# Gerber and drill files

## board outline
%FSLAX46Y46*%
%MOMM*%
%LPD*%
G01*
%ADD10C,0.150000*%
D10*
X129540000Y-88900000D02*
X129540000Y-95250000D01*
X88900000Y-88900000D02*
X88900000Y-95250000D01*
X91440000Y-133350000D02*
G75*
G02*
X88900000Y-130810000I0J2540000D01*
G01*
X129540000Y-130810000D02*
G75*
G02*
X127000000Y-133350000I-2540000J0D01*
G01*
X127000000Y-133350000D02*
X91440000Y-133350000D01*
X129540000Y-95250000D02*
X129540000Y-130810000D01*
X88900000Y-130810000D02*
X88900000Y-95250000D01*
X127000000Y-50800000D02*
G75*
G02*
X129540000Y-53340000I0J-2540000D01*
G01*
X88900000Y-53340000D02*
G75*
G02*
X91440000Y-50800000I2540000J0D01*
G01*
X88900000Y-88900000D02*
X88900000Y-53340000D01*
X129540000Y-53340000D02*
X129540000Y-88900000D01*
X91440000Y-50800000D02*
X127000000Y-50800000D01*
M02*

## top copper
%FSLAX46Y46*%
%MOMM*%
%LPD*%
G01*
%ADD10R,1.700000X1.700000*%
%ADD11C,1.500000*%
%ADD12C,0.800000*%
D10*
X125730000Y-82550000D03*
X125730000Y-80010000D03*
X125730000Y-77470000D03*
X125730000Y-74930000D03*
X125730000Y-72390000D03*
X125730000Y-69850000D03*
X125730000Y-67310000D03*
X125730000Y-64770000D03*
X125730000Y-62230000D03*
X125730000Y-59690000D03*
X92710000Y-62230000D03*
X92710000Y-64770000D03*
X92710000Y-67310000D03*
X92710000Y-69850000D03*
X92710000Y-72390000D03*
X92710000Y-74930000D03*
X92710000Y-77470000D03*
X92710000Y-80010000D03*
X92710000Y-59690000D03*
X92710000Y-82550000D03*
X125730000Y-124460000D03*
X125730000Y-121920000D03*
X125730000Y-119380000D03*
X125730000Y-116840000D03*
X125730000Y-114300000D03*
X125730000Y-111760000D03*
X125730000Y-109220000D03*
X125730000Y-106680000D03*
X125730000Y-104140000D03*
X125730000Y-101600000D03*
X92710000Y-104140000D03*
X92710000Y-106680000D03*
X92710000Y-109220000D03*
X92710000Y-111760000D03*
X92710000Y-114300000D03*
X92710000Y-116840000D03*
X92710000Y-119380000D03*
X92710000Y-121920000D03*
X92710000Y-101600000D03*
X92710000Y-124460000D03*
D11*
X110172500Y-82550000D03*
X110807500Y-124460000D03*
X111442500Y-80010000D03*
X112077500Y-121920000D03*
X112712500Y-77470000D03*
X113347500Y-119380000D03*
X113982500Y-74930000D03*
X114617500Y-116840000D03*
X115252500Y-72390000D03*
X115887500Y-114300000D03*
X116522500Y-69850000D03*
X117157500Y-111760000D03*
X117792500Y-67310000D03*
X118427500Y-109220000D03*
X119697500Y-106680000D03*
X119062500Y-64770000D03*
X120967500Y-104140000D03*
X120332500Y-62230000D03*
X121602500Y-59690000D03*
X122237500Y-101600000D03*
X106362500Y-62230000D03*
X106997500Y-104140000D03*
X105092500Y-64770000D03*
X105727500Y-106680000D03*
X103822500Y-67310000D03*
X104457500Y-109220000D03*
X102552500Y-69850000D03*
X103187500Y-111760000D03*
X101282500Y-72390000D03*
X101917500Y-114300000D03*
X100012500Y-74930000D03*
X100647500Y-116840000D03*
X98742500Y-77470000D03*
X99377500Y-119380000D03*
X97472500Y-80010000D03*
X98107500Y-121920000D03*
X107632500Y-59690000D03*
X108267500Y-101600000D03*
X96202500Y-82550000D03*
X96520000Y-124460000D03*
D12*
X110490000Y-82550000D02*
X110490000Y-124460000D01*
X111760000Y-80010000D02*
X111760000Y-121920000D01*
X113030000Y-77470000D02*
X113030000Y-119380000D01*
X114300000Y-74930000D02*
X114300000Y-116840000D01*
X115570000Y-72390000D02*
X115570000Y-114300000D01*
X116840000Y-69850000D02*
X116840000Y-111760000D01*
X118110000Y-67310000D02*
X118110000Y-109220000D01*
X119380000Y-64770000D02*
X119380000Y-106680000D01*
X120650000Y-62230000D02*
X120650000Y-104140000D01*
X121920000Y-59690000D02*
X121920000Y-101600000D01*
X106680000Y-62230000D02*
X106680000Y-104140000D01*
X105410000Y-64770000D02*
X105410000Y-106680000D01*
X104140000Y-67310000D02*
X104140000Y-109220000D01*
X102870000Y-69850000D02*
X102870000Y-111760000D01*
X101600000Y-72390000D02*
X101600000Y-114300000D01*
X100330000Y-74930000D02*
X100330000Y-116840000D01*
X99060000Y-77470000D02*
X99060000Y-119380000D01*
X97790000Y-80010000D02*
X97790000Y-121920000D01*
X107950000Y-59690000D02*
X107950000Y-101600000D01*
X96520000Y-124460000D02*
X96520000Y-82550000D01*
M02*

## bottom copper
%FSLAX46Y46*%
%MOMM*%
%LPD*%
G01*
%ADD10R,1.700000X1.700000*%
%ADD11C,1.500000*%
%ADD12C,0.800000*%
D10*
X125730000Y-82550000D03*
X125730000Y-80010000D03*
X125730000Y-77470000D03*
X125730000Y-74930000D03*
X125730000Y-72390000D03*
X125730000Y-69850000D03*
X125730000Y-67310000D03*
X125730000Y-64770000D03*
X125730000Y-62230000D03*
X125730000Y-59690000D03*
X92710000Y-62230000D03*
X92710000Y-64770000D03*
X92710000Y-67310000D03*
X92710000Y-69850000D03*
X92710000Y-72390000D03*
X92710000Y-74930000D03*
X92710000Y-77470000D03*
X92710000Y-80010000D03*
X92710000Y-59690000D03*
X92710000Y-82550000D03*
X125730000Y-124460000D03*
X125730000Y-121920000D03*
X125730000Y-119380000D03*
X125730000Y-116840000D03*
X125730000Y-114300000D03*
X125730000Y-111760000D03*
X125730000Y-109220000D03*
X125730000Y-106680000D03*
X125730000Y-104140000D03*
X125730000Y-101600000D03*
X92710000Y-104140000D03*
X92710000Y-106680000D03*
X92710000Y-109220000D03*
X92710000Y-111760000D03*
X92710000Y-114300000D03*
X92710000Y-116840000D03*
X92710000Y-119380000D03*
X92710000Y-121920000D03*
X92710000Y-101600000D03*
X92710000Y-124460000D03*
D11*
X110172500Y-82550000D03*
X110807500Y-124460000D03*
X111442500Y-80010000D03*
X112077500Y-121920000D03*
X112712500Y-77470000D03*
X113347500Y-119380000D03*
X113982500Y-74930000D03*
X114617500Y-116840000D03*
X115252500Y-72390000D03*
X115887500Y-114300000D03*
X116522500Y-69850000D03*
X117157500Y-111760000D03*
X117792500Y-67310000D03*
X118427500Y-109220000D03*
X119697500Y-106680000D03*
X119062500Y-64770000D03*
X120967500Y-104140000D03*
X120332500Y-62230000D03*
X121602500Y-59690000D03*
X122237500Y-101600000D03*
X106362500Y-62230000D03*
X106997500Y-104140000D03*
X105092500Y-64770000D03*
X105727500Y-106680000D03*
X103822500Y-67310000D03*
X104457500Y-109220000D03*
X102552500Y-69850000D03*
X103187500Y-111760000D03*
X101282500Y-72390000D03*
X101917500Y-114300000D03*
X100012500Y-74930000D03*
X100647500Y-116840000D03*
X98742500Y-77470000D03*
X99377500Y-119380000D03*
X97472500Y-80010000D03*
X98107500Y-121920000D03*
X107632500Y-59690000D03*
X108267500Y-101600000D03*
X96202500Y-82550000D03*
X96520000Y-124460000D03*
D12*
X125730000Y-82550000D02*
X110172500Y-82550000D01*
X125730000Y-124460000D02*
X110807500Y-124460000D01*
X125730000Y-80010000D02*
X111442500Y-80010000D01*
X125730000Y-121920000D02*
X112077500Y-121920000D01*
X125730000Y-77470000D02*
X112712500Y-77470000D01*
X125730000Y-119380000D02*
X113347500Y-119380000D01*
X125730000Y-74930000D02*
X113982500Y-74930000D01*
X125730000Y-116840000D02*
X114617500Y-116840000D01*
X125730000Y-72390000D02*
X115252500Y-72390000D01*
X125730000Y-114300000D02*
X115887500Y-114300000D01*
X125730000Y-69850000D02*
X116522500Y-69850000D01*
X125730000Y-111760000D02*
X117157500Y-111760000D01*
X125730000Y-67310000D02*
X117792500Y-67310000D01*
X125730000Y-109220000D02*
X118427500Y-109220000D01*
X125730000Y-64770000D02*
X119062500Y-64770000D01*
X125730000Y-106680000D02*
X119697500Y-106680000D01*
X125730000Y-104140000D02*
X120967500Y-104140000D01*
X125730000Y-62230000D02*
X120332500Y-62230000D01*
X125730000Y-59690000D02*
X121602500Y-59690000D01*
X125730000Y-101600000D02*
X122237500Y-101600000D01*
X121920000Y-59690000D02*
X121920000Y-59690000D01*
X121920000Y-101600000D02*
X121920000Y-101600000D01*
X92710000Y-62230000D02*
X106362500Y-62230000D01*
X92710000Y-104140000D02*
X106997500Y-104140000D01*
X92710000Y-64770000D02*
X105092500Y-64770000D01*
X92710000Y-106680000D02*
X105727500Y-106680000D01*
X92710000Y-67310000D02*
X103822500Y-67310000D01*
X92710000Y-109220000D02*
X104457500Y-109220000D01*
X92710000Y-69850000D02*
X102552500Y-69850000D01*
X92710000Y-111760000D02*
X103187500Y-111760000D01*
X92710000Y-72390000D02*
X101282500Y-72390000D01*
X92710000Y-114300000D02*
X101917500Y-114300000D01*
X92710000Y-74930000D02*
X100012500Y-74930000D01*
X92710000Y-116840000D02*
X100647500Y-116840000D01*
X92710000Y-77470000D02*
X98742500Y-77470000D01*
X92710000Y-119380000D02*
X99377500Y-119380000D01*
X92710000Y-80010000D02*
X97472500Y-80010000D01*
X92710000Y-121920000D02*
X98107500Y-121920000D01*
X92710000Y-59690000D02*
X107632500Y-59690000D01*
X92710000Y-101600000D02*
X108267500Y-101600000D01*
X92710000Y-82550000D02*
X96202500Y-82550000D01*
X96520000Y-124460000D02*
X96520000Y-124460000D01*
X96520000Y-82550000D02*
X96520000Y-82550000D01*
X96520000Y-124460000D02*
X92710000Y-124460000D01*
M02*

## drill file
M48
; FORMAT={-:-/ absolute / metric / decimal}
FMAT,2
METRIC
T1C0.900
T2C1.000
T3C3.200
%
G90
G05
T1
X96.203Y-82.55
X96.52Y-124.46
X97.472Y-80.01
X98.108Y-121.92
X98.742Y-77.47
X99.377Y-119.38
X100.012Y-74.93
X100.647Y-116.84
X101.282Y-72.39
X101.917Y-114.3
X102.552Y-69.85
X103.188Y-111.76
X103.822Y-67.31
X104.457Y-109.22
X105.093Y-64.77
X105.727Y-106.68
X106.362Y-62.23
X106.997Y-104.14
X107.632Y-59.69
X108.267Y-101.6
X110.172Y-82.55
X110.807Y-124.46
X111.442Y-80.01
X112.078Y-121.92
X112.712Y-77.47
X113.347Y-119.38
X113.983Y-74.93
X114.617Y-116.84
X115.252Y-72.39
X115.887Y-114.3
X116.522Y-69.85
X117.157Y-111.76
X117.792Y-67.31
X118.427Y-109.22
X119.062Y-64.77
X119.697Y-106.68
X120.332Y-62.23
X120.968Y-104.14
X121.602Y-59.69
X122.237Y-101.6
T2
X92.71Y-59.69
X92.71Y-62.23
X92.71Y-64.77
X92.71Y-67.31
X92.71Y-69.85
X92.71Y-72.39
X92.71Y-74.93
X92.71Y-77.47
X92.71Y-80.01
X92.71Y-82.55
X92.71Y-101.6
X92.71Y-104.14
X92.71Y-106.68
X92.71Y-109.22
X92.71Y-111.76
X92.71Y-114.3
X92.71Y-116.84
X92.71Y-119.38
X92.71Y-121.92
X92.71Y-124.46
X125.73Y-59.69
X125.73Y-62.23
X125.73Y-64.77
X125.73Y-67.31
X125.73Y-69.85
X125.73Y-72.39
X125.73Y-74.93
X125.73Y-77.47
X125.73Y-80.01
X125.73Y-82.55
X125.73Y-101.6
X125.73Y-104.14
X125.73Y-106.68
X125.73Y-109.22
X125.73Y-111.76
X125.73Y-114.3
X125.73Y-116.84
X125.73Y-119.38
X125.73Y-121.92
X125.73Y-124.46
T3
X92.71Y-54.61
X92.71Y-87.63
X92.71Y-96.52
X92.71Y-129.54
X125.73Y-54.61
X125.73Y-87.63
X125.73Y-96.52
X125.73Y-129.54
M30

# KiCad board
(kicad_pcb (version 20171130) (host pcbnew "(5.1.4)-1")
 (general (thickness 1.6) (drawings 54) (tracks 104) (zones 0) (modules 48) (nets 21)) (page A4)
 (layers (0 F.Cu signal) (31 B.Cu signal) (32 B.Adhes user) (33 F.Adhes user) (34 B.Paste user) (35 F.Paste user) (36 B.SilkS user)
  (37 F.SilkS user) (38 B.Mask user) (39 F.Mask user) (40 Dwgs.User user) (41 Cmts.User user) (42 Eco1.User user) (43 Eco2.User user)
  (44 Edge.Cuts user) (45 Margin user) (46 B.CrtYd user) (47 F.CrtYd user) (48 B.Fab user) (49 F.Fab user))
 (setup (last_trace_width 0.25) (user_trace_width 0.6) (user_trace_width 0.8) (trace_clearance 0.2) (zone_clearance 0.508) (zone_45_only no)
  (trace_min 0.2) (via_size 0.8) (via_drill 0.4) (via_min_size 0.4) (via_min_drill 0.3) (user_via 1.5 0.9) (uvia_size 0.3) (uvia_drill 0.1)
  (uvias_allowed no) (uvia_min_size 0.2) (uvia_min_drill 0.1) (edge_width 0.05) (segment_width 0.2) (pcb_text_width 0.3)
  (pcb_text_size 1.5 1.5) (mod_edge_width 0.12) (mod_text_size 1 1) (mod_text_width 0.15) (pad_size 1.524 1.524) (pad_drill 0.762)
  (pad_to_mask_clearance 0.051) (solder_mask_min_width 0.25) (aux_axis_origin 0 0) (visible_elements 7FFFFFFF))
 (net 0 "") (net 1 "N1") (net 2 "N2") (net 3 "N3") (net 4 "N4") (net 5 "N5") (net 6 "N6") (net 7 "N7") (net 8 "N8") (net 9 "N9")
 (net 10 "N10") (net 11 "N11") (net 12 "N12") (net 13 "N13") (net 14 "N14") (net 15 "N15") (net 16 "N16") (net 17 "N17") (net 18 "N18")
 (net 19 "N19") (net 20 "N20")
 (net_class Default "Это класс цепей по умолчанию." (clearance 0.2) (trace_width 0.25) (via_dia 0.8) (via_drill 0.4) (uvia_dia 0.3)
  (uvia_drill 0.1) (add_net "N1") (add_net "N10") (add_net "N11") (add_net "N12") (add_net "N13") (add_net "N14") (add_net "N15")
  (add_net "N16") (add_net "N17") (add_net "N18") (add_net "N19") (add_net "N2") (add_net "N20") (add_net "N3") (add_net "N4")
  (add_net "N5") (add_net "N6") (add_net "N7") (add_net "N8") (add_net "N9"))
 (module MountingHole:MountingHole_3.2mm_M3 (layer F.Cu) (at 92.71 129.54)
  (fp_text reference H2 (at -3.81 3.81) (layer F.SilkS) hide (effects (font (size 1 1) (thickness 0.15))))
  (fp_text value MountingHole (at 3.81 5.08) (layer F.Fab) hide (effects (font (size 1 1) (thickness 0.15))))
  (pad 1 np_thru_hole circle (at 0 0) (size 3.2 3.2) (drill 3.2) (layers *.Cu *.Mask)))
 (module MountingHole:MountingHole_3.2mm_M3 (layer F.Cu) (at 125.73 129.54)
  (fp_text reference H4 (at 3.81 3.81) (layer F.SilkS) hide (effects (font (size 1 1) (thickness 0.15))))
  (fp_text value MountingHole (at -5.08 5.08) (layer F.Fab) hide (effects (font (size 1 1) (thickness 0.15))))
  (pad 1 np_thru_hole circle (at 0 0) (size 3.2 3.2) (drill 3.2) (layers *.Cu *.Mask)))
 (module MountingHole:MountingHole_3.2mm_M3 (layer F.Cu) (at 92.71 96.52)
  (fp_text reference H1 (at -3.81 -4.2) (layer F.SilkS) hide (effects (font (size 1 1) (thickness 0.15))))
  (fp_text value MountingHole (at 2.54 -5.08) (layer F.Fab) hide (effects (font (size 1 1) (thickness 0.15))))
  (pad 1 np_thru_hole circle (at 0 0) (size 3.2 3.2) (drill 3.2) (layers *.Cu *.Mask)))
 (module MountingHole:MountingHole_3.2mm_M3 (layer F.Cu) (at 125.73 96.52)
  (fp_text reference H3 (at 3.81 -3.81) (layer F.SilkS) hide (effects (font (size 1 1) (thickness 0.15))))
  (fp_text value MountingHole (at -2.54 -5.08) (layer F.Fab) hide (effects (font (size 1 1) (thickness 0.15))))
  (pad 1 np_thru_hole circle (at 0 0) (size 3.2 3.2) (drill 3.2) (layers *.Cu *.Mask)))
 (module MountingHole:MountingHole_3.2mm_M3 (layer F.Cu) (at 92.71 54.61)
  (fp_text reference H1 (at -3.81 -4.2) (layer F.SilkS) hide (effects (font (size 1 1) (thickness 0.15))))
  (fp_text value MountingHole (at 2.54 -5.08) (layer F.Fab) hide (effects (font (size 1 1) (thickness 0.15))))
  (pad 1 np_thru_hole circle (at 0 0) (size 3.2 3.2) (drill 3.2) (layers *.Cu *.Mask)))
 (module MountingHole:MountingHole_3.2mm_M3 (layer F.Cu) (at 92.71 87.63)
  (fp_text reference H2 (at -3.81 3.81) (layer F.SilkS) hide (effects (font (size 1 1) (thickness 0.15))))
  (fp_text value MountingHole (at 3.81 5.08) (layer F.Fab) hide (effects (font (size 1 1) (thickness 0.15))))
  (pad 1 np_thru_hole circle (at 0 0) (size 3.2 3.2) (drill 3.2) (layers *.Cu *.Mask)))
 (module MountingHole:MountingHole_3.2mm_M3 (layer F.Cu) (at 125.73 54.61)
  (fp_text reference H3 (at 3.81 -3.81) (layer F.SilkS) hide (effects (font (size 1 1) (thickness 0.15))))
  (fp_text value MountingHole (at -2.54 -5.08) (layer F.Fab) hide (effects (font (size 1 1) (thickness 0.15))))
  (pad 1 np_thru_hole circle (at 0 0) (size 3.2 3.2) (drill 3.2) (layers *.Cu *.Mask)))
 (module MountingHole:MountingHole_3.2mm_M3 (layer F.Cu) (at 125.73 87.63)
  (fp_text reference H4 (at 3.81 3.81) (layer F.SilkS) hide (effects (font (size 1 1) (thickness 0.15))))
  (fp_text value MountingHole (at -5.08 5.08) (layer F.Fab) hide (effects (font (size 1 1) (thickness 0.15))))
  (pad 1 np_thru_hole circle (at 0 0) (size 3.2 3.2) (drill 3.2) (layers *.Cu *.Mask)))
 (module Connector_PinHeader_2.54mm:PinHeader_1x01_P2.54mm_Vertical (layer F.Cu) (at 125.73 82.55)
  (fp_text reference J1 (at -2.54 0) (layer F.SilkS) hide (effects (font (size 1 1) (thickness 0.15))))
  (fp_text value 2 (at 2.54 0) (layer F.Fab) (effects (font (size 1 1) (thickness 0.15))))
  (pad 1 thru_hole rect (at 0 0) (size 1.7 1.7) (drill 1) (layers *.Cu *.Mask) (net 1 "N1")))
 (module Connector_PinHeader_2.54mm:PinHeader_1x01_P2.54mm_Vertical (layer F.Cu) (at 125.73 80.01)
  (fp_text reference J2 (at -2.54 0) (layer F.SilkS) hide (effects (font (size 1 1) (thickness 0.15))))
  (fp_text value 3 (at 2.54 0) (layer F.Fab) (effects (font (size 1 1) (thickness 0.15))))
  (pad 1 thru_hole rect (at 0 0) (size 1.7 1.7) (drill 1) (layers *.Cu *.Mask) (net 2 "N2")))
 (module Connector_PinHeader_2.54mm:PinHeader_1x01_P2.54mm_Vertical (layer F.Cu) (at 125.73 77.47)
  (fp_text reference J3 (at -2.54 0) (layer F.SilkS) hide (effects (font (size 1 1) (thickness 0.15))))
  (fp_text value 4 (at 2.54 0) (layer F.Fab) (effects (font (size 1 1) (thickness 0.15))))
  (pad 1 thru_hole rect (at 0 0) (size 1.7 1.7) (drill 1) (layers *.Cu *.Mask) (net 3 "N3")))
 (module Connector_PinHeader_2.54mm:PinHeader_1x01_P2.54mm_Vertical (layer F.Cu) (at 125.73 74.93)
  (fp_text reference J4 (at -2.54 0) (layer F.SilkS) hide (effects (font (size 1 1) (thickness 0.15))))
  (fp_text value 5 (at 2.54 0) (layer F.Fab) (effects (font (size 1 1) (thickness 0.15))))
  (pad 1 thru_hole rect (at 0 0) (size 1.7 1.7) (drill 1) (layers *.Cu *.Mask) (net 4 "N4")))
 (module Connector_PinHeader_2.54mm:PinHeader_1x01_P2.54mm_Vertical (layer F.Cu) (at 125.73 72.39)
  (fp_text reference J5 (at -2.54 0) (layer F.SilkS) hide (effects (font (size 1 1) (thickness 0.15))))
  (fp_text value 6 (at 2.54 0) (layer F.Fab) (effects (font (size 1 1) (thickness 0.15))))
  (pad 1 thru_hole rect (at 0 0) (size 1.7 1.7) (drill 1) (layers *.Cu *.Mask) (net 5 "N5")))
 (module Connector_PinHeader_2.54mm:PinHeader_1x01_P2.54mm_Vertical (layer F.Cu) (at 125.73 69.85)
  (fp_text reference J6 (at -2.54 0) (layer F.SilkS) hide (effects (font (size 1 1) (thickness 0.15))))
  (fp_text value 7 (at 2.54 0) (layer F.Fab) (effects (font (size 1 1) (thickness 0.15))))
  (pad 1 thru_hole rect (at 0 0) (size 1.7 1.7) (drill 1) (layers *.Cu *.Mask) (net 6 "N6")))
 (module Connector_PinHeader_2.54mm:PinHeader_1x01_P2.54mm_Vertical (layer F.Cu) (at 125.73 67.31)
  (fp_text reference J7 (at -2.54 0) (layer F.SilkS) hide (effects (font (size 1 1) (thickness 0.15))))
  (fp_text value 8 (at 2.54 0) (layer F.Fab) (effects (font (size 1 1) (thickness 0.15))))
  (pad 1 thru_hole rect (at 0 0) (size 1.7 1.7) (drill 1) (layers *.Cu *.Mask) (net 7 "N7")))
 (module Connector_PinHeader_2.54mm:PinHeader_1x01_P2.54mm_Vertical (layer F.Cu) (at 125.73 64.77)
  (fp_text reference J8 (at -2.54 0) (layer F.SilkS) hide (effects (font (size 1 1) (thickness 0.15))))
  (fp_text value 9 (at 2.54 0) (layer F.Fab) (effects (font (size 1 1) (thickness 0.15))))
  (pad 1 thru_hole rect (at 0 0) (size 1.7 1.7) (drill 1) (layers *.Cu *.Mask) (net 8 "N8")))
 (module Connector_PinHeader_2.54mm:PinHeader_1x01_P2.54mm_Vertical (layer F.Cu) (at 125.73 62.23)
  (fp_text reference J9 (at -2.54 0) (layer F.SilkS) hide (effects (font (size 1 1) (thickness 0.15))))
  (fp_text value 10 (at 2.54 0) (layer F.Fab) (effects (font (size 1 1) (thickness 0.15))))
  (pad 1 thru_hole rect (at 0 0) (size 1.7 1.7) (drill 1) (layers *.Cu *.Mask) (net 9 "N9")))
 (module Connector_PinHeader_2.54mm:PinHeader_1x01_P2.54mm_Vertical (layer F.Cu) (at 125.73 59.69)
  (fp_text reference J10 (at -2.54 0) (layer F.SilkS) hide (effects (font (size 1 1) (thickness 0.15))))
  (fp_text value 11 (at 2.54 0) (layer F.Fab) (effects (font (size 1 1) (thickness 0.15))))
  (pad 1 thru_hole rect (at 0 0) (size 1.7 1.7) (drill 1) (layers *.Cu *.Mask) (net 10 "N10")))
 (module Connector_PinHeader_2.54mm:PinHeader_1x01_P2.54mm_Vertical (layer F.Cu) (at 92.71 62.23)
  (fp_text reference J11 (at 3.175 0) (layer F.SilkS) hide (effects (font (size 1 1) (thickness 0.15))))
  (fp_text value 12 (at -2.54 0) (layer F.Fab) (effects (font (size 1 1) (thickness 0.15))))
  (pad 1 thru_hole rect (at 0 0) (size 1.7 1.7) (drill 1) (layers *.Cu *.Mask) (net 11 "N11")))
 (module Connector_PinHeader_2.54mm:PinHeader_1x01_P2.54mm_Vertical (layer F.Cu) (at 92.71 64.77)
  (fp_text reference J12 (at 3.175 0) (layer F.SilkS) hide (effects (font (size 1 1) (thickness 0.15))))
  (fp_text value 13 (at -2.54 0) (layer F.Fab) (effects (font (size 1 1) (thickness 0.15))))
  (pad 1 thru_hole rect (at 0 0) (size 1.7 1.7) (drill 1) (layers *.Cu *.Mask) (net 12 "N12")))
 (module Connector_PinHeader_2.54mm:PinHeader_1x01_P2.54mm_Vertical (layer F.Cu) (at 92.71 67.31)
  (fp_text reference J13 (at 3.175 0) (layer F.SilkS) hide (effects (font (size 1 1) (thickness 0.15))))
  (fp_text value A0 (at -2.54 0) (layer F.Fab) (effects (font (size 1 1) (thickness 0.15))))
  (pad 1 thru_hole rect (at 0 0) (size 1.7 1.7) (drill 1) (layers *.Cu *.Mask) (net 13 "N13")))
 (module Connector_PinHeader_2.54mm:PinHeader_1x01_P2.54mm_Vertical (layer F.Cu) (at 92.71 69.85)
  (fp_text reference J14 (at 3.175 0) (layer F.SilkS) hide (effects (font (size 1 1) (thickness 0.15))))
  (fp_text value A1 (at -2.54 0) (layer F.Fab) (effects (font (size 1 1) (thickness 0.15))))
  (pad 1 thru_hole rect (at 0 0) (size 1.7 1.7) (drill 1) (layers *.Cu *.Mask) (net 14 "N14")))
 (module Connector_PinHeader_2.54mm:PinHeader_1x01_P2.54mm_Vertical (layer F.Cu) (at 92.71 72.39)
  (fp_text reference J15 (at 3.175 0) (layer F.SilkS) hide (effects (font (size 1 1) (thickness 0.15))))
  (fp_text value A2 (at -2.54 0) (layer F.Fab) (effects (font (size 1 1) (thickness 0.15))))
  (pad 1 thru_hole rect (at 0 0) (size 1.7 1.7) (drill 1) (layers *.Cu *.Mask) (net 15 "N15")))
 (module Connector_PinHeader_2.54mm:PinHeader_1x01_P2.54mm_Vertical (layer F.Cu) (at 92.71 74.93)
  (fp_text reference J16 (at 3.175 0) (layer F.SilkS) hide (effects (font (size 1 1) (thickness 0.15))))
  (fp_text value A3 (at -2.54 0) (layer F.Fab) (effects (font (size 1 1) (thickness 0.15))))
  (pad 1 thru_hole rect (at 0 0) (size 1.7 1.7) (drill 1) (layers *.Cu *.Mask) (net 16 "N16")))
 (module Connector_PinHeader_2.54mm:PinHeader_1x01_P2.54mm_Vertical (layer F.Cu) (at 92.71 77.47)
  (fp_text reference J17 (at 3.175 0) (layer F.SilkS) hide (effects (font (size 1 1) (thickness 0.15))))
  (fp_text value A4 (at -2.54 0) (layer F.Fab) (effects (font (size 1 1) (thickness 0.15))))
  (pad 1 thru_hole rect (at 0 0) (size 1.7 1.7) (drill 1) (layers *.Cu *.Mask) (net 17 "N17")))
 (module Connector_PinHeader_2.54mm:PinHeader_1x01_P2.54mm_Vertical (layer F.Cu) (at 92.71 80.01)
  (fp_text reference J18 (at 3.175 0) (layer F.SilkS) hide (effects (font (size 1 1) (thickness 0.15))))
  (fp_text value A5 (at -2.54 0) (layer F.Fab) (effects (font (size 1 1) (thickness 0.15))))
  (pad 1 thru_hole rect (at 0 0) (size 1.7 1.7) (drill 1) (layers *.Cu *.Mask) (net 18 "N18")))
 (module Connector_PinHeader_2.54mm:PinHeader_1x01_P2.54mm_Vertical (layer F.Cu) (at 92.71 59.69)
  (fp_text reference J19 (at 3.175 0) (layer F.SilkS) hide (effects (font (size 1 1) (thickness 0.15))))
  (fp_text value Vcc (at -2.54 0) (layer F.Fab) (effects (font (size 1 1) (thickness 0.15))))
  (pad 1 thru_hole rect (at 0 0) (size 1.7 1.7) (drill 1) (layers *.Cu *.Mask) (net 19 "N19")))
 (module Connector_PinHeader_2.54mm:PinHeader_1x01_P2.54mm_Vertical (layer F.Cu) (at 92.71 82.55)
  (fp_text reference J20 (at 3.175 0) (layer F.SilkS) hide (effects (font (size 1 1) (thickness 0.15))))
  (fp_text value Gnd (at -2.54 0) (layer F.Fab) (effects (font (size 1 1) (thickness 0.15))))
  (pad 1 thru_hole rect (at 0 0) (size 1.7 1.7) (drill 1) (layers *.Cu *.Mask) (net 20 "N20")))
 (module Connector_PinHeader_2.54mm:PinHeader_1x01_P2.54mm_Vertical (layer F.Cu) (at 125.73 124.46)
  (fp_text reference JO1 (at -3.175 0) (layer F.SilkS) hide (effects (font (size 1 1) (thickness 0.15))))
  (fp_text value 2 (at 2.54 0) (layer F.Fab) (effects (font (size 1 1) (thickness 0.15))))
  (pad 1 thru_hole rect (at 0 0) (size 1.7 1.7) (drill 1) (layers *.Cu *.Mask) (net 1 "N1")))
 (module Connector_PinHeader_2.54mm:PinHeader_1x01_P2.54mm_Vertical (layer F.Cu) (at 125.73 121.92)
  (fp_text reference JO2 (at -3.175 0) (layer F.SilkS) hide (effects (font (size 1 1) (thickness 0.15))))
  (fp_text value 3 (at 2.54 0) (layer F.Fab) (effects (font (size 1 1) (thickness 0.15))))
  (pad 1 thru_hole rect (at 0 0) (size 1.7 1.7) (drill 1) (layers *.Cu *.Mask) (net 2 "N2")))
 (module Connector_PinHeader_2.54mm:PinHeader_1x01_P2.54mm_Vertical (layer F.Cu) (at 125.73 119.38)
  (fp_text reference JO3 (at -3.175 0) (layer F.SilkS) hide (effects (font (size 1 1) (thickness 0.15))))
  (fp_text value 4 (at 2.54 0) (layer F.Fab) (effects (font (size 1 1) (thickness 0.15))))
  (pad 1 thru_hole rect (at 0 0) (size 1.7 1.7) (drill 1) (layers *.Cu *.Mask) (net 3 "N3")))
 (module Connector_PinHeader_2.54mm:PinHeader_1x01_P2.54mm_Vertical (layer F.Cu) (at 125.73 116.84)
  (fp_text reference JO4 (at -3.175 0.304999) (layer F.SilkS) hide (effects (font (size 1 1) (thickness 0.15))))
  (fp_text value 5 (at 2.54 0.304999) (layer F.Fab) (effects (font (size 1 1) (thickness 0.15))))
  (pad 1 thru_hole rect (at 0 0) (size 1.7 1.7) (drill 1) (layers *.Cu *.Mask) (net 4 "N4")))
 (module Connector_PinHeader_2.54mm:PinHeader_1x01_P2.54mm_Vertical (layer F.Cu) (at 125.73 114.3)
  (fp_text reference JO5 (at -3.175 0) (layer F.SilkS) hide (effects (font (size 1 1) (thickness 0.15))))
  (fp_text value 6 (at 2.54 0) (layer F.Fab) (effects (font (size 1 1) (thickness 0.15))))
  (pad 1 thru_hole rect (at 0 0) (size 1.7 1.7) (drill 1) (layers *.Cu *.Mask) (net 5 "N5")))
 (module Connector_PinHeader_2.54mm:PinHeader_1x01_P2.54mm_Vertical (layer F.Cu) (at 125.73 111.76)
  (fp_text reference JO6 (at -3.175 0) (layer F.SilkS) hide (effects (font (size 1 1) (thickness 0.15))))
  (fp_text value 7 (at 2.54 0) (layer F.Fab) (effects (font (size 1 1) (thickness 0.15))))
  (pad 1 thru_hole rect (at 0 0) (size 1.7 1.7) (drill 1) (layers *.Cu *.Mask) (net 6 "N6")))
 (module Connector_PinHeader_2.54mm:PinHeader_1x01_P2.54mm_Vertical (layer F.Cu) (at 125.73 109.22)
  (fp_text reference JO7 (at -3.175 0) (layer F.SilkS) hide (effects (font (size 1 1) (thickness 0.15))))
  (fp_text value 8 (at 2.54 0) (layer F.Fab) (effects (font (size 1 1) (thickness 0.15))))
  (pad 1 thru_hole rect (at 0 0) (size 1.7 1.7) (drill 1) (layers *.Cu *.Mask) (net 7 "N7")))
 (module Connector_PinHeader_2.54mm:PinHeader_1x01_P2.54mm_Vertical (layer F.Cu) (at 125.73 106.68)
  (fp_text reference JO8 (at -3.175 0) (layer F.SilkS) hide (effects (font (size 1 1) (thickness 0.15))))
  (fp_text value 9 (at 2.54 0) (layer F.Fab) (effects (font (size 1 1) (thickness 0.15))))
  (pad 1 thru_hole rect (at 0 0) (size 1.7 1.7) (drill 1) (layers *.Cu *.Mask) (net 8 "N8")))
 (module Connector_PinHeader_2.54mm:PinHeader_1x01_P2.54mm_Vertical (layer F.Cu) (at 125.73 104.14)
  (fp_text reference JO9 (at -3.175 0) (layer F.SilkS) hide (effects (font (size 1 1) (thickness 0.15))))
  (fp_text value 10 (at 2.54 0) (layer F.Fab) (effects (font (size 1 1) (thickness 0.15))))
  (pad 1 thru_hole rect (at 0 0) (size 1.7 1.7) (drill 1) (layers *.Cu *.Mask) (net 9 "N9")))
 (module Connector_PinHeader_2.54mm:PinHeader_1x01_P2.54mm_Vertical (layer F.Cu) (at 125.73 101.6)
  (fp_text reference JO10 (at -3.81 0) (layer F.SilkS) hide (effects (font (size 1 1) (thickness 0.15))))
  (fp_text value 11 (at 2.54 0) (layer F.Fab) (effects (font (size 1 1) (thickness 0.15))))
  (pad 1 thru_hole rect (at 0 0) (size 1.7 1.7) (drill 1) (layers *.Cu *.Mask) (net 10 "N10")))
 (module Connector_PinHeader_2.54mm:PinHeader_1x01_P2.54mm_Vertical (layer F.Cu) (at 92.71 104.14)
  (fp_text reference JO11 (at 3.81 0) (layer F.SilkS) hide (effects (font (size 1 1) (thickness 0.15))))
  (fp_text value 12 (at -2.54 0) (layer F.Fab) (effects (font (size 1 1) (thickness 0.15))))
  (pad 1 thru_hole rect (at 0 0) (size 1.7 1.7) (drill 1) (layers *.Cu *.Mask) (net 11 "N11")))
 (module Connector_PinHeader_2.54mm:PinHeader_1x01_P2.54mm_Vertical (layer F.Cu) (at 92.71 106.68)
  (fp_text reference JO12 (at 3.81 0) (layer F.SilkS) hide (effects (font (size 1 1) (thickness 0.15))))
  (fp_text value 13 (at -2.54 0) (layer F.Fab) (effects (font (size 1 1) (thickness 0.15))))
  (pad 1 thru_hole rect (at 0 0) (size 1.7 1.7) (drill 1) (layers *.Cu *.Mask) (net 12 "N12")))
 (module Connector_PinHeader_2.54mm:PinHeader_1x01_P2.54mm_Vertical (layer F.Cu) (at 92.71 109.22)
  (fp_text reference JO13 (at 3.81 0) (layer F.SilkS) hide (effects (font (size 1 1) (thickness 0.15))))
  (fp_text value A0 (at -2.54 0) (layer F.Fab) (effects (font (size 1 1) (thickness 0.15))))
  (pad 1 thru_hole rect (at 0 0) (size 1.7 1.7) (drill 1) (layers *.Cu *.Mask) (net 13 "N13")))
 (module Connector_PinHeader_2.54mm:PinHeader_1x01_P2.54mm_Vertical (layer F.Cu) (at 92.71 111.76)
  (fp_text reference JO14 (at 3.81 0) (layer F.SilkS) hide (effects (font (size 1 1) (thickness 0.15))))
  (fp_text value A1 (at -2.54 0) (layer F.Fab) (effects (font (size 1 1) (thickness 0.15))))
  (pad 1 thru_hole rect (at 0 0) (size 1.7 1.7) (drill 1) (layers *.Cu *.Mask) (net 14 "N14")))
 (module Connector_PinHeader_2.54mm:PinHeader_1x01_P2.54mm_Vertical (layer F.Cu) (at 92.71 114.3)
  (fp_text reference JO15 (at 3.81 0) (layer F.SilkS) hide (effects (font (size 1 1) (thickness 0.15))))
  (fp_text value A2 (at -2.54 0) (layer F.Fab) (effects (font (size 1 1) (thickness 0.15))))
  (pad 1 thru_hole rect (at 0 0) (size 1.7 1.7) (drill 1) (layers *.Cu *.Mask) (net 15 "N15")))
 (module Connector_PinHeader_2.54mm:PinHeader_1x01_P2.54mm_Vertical (layer F.Cu) (at 92.71 116.84)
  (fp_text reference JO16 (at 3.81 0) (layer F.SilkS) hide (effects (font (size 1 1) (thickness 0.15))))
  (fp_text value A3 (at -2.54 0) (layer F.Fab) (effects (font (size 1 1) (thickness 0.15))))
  (pad 1 thru_hole rect (at 0 0) (size 1.7 1.7) (drill 1) (layers *.Cu *.Mask) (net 16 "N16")))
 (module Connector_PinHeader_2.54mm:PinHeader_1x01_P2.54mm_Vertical (layer F.Cu) (at 92.71 119.38)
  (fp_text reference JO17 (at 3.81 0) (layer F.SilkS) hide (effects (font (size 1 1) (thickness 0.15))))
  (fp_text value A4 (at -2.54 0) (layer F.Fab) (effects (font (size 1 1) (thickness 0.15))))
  (pad 1 thru_hole rect (at 0 0) (size 1.7 1.7) (drill 1) (layers *.Cu *.Mask) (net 17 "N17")))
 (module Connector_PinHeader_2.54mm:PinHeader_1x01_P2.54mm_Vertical (layer F.Cu) (at 92.71 121.92)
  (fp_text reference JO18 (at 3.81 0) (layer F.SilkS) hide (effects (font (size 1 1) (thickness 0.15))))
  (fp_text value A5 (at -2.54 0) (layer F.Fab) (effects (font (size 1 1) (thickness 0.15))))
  (pad 1 thru_hole rect (at 0 0) (size 1.7 1.7) (drill 1) (layers *.Cu *.Mask) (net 18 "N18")))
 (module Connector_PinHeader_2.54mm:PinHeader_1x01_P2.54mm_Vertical (layer F.Cu) (at 92.71 101.6)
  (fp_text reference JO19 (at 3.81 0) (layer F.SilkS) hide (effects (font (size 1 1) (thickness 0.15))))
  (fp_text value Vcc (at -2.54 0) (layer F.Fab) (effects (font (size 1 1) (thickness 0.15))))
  (pad 1 thru_hole rect (at 0 0) (size 1.7 1.7) (drill 1) (layers *.Cu *.Mask) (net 19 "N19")))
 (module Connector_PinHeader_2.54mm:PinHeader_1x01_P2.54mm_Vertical (layer F.Cu) (at 92.71 124.46)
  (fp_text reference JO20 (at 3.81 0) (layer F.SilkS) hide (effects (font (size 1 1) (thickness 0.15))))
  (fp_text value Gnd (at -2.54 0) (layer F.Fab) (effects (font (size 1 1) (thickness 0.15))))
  (pad 1 thru_hole rect (at 0 0) (size 1.7 1.7) (drill 1) (layers *.Cu *.Mask) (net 20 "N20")))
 (gr_line (start 129.54 88.9) (end 129.54 95.25) (layer Edge.Cuts) (width 0.15))
 (gr_line (start 88.9 88.9) (end 88.9 95.25) (layer Edge.Cuts) (width 0.15))
 (gr_arc (start 91.44 130.81) (end 88.9 130.81) (angle -90) (layer Edge.Cuts) (width 0.15))
 (gr_arc (start 127 130.81) (end 127 133.35) (angle -90) (layer Edge.Cuts) (width 0.15))
 (gr_line (start 127 133.35) (end 91.44 133.35) (layer Edge.Cuts) (width 0.15))
 (gr_line (start 129.54 95.25) (end 129.54 130.81) (layer Edge.Cuts) (width 0.15))
 (gr_line (start 88.9 130.81) (end 88.9 95.25) (layer Edge.Cuts) (width 0.15))
 (gr_arc (start 127 53.34) (end 129.54 53.34) (angle -90) (layer Edge.Cuts) (width 0.15))
 (gr_arc (start 91.44 53.34) (end 91.44 50.8) (angle -90) (layer Edge.Cuts) (width 0.15))
 (gr_line (start 88.9 88.9) (end 88.9 53.34) (layer Edge.Cuts) (width 0.15))
 (gr_line (start 129.54 53.34) (end 129.54 88.9) (layer Edge.Cuts) (width 0.15))
 (gr_line (start 91.44 50.8) (end 127 50.8) (layer Edge.Cuts) (width 0.15))
 (segment (start 125.73 82.55) (end 110.1725 82.55) (width 0.8) (layer B.Cu) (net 1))
 (via (at 110.1725 82.55) (size 1.5) (drill 0.9) (layers F.Cu B.Cu) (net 1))
 (segment (start 125.73 124.46) (end 110.8075 124.46) (width 0.8) (layer B.Cu) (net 1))
 (via (at 110.8075 124.46) (size 1.5) (drill 0.9) (layers F.Cu B.Cu) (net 1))
 (segment (start 110.49 82.55) (end 110.49 124.46) (width 0.8) (layer F.Cu) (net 1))
 (segment (start 125.73 80.01) (end 111.4425 80.01) (width 0.8) (layer B.Cu) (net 2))
 (via (at 111.4425 80.01) (size 1.5) (drill 0.9) (layers F.Cu B.Cu) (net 2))
 (segment (start 125.73 121.92) (end 112.0775 121.92) (width 0.8) (layer B.Cu) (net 2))
 (via (at 112.0775 121.92) (size 1.5) (drill 0.9) (layers F.Cu B.Cu) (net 2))
 (segment (start 111.76 80.01) (end 111.76 121.92) (width 0.8) (layer F.Cu) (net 2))
 (segment (start 125.73 77.47) (end 112.7125 77.47) (width 0.8) (layer B.Cu) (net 3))
 (via (at 112.7125 77.47) (size 1.5) (drill 0.9) (layers F.Cu B.Cu) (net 3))
 (segment (start 125.73 119.38) (end 113.3475 119.38) (width 0.8) (layer B.Cu) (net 3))
 (via (at 113.3475 119.38) (size 1.5) (drill 0.9) (layers F.Cu B.Cu) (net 3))
 (segment (start 113.03 77.47) (end 113.03 119.38) (width 0.8) (layer F.Cu) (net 3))
 (segment (start 125.73 74.93) (end 113.9825 74.93) (width 0.8) (layer B.Cu) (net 4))
 (via (at 113.9825 74.93) (size 1.5) (drill 0.9) (layers F.Cu B.Cu) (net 4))
 (segment (start 125.73 116.84) (end 114.6175 116.84) (width 0.8) (layer B.Cu) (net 4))
 (via (at 114.6175 116.84) (size 1.5) (drill 0.9) (layers F.Cu B.Cu) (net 4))
 (segment (start 114.3 74.93) (end 114.3 116.84) (width 0.8) (layer F.Cu) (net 4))
 (segment (start 125.73 72.39) (end 115.2525 72.39) (width 0.8) (layer B.Cu) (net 5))
 (via (at 115.2525 72.39) (size 1.5) (drill 0.9) (layers F.Cu B.Cu) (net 5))
 (segment (start 125.73 114.3) (end 115.8875 114.3) (width 0.8) (layer B.Cu) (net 5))
 (via (at 115.8875 114.3) (size 1.5) (drill 0.9) (layers F.Cu B.Cu) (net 5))
 (segment (start 115.57 72.39) (end 115.57 114.3) (width 0.8) (layer F.Cu) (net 5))
 (segment (start 125.73 69.85) (end 116.5225 69.85) (width 0.8) (layer B.Cu) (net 6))
 (via (at 116.5225 69.85) (size 1.5) (drill 0.9) (layers F.Cu B.Cu) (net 6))
 (segment (start 125.73 111.76) (end 117.1575 111.76) (width 0.8) (layer B.Cu) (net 6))
 (via (at 117.1575 111.76) (size 1.5) (drill 0.9) (layers F.Cu B.Cu) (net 6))
 (segment (start 116.84 69.85) (end 116.84 111.76) (width 0.8) (layer F.Cu) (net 6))
 (segment (start 125.73 67.31) (end 117.7925 67.31) (width 0.8) (layer B.Cu) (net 7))
 (via (at 117.7925 67.31) (size 1.5) (drill 0.9) (layers F.Cu B.Cu) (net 7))
 (segment (start 125.73 109.22) (end 118.4275 109.22) (width 0.8) (layer B.Cu) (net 7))
 (via (at 118.4275 109.22) (size 1.5) (drill 0.9) (layers F.Cu B.Cu) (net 7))
 (segment (start 118.11 67.31) (end 118.11 109.22) (width 0.8) (layer F.Cu) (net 7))
 (segment (start 125.73 64.77) (end 119.0625 64.77) (width 0.8) (layer B.Cu) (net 8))
 (segment (start 125.73 106.68) (end 119.6975 106.68) (width 0.8) (layer B.Cu) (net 8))
 (via (at 119.6975 106.68) (size 1.5) (drill 0.9) (layers F.Cu B.Cu) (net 8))
 (via (at 119.0625 64.77) (size 1.5) (drill 0.9) (layers F.Cu B.Cu) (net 8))
 (segment (start 119.38 64.77) (end 119.38 106.68) (width 0.8) (layer F.Cu) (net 8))
 (via (at 120.9675 104.14) (size 1.5) (drill 0.9) (layers F.Cu B.Cu) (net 9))
 (segment (start 125.73 104.14) (end 120.9675 104.14) (width 0.8) (layer B.Cu) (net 9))
 (segment (start 125.73 62.23) (end 120.3325 62.23) (width 0.8) (layer B.Cu) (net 9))
 (via (at 120.3325 62.23) (size 1.5) (drill 0.9) (layers F.Cu B.Cu) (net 9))
 (segment (start 120.65 62.23) (end 120.65 104.14) (width 0.8) (layer F.Cu) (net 9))
 (segment (start 125.73 59.69) (end 121.6025 59.69) (width 0.8) (layer B.Cu) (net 10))
 (segment (start 125.73 101.6) (end 122.2375 101.6) (width 0.8) (layer B.Cu) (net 10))
 (segment (start 121.92 59.69) (end 121.92 59.69) (width 0.8) (layer B.Cu) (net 10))
 (via (at 121.6025 59.69) (size 1.5) (drill 0.9) (layers F.Cu B.Cu) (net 10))
 (segment (start 121.92 101.6) (end 121.92 101.6) (width 0.8) (layer B.Cu) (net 10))
 (via (at 122.2375 101.6) (size 1.5) (drill 0.9) (layers F.Cu B.Cu) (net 10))
 (segment (start 121.92 59.69) (end 121.92 101.6) (width 0.8) (layer F.Cu) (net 10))
 (via (at 106.3625 62.23) (size 1.5) (drill 0.9) (layers F.Cu B.Cu) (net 11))
 (segment (start 106.68 62.23) (end 106.68 104.14) (width 0.8) (layer F.Cu) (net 11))
 (via (at 106.9975 104.14) (size 1.5) (drill 0.9) (layers F.Cu B.Cu) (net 11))
 (segment (start 92.71 62.23) (end 106.3625 62.23) (width 0.8) (layer B.Cu) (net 11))
 (segment (start 92.71 104.14) (end 106.9975 104.14) (width 0.8) (layer B.Cu) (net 11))
 (via (at 105.0925 64.77) (size 1.5) (drill 0.9) (layers F.Cu B.Cu) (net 12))
 (segment (start 105.41 64.77) (end 105.41 106.68) (width 0.8) (layer F.Cu) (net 12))
 (via (at 105.7275 106.68) (size 1.5) (drill 0.9) (layers F.Cu B.Cu) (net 12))
 (segment (start 92.71 64.77) (end 105.0925 64.77) (width 0.8) (layer B.Cu) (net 12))
 (segment (start 92.71 106.68) (end 105.7275 106.68) (width 0.8) (layer B.Cu) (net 12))
 (via (at 103.8225 67.31) (size 1.5) (drill 0.9) (layers F.Cu B.Cu) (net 13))
 (segment (start 104.14 67.31) (end 104.14 109.22) (width 0.8) (layer F.Cu) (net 13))
 (via (at 104.4575 109.22) (size 1.5) (drill 0.9) (layers F.Cu B.Cu) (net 13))
 (segment (start 92.71 67.31) (end 103.8225 67.31) (width 0.8) (layer B.Cu) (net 13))
 (segment (start 92.71 109.22) (end 104.4575 109.22) (width 0.8) (layer B.Cu) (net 13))
 (via (at 102.5525 69.85) (size 1.5) (drill 0.9) (layers F.Cu B.Cu) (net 14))
 (segment (start 102.87 69.85) (end 102.87 111.76) (width 0.8) (layer F.Cu) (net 14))
 (via (at 103.1875 111.76) (size 1.5) (drill 0.9) (layers F.Cu B.Cu) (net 14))
 (segment (start 92.71 69.85) (end 102.5525 69.85) (width 0.8) (layer B.Cu) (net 14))
 (segment (start 92.71 111.76) (end 103.1875 111.76) (width 0.8) (layer B.Cu) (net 14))
 (via (at 101.2825 72.39) (size 1.5) (drill 0.9) (layers F.Cu B.Cu) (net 15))
 (segment (start 101.6 72.39) (end 101.6 114.3) (width 0.8) (layer F.Cu) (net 15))
 (via (at 101.9175 114.3) (size 1.5) (drill 0.9) (layers F.Cu B.Cu) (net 15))
 (segment (start 92.71 72.39) (end 101.2825 72.39) (width 0.8) (layer B.Cu) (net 15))
 (segment (start 92.71 114.3) (end 101.9175 114.3) (width 0.8) (layer B.Cu) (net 15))
 (via (at 100.0125 74.93) (size 1.5) (drill 0.9) (layers F.Cu B.Cu) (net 16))
 (segment (start 100.33 74.93) (end 100.33 116.84) (width 0.8) (layer F.Cu) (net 16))
 (via (at 100.6475 116.84) (size 1.5) (drill 0.9) (layers F.Cu B.Cu) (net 16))
 (segment (start 92.71 74.93) (end 100.0125 74.93) (width 0.8) (layer B.Cu) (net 16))
 (segment (start 92.71 116.84) (end 100.6475 116.84) (width 0.8) (layer B.Cu) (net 16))
 (via (at 98.7425 77.47) (size 1.5) (drill 0.9) (layers F.Cu B.Cu) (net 17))
 (segment (start 99.06 77.47) (end 99.06 119.38) (width 0.8) (layer F.Cu) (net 17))
 (via (at 99.3775 119.38) (size 1.5) (drill 0.9) (layers F.Cu B.Cu) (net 17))
 (segment (start 92.71 77.47) (end 98.7425 77.47) (width 0.8) (layer B.Cu) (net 17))
 (segment (start 92.71 119.38) (end 99.3775 119.38) (width 0.8) (layer B.Cu) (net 17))
 (via (at 97.4725 80.01) (size 1.5) (drill 0.9) (layers F.Cu B.Cu) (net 18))
 (via (at 98.1075 121.92) (size 1.5) (drill 0.9) (layers F.Cu B.Cu) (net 18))
 (segment (start 97.79 80.01) (end 97.79 121.92) (width 0.8) (layer F.Cu) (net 18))
 (segment (start 92.71 80.01) (end 97.4725 80.01) (width 0.8) (layer B.Cu) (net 18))
 (segment (start 92.71 121.92) (end 98.1075 121.92) (width 0.8) (layer B.Cu) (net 18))
 (via (at 107.6325 59.69) (size 1.5) (drill 0.9) (layers F.Cu B.Cu) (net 19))
 (segment (start 107.95 59.69) (end 107.95 101.6) (width 0.8) (layer F.Cu) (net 19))
 (via (at 108.2675 101.6) (size 1.5) (drill 0.9) (layers F.Cu B.Cu) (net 19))
 (segment (start 92.71 59.69) (end 107.6325 59.69) (width 0.8) (layer B.Cu) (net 19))
 (segment (start 92.71 101.6) (end 108.2675 101.6) (width 0.8) (layer B.Cu) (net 19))
 (segment (start 92.71 82.55) (end 96.2025 82.55) (width 0.8) (layer B.Cu) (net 20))
 (segment (start 96.52 124.46) (end 96.52 82.55) (width 0.8) (layer F.Cu) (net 20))
 (segment (start 96.52 124.46) (end 96.52 124.46) (width 0.8) (layer B.Cu) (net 20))
 (segment (start 96.52 82.55) (end 96.52 82.55) (width 0.8) (layer B.Cu) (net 20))
 (via (at 96.2025 82.55) (size 1.5) (drill 0.9) (layers F.Cu B.Cu) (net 20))
 (segment (start 96.52 124.46) (end 92.71 124.46) (width 0.8) (layer B.Cu) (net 20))
 (via (at 96.52 124.46) (size 1.5) (drill 0.9) (layers F.Cu B.Cu) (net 20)))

